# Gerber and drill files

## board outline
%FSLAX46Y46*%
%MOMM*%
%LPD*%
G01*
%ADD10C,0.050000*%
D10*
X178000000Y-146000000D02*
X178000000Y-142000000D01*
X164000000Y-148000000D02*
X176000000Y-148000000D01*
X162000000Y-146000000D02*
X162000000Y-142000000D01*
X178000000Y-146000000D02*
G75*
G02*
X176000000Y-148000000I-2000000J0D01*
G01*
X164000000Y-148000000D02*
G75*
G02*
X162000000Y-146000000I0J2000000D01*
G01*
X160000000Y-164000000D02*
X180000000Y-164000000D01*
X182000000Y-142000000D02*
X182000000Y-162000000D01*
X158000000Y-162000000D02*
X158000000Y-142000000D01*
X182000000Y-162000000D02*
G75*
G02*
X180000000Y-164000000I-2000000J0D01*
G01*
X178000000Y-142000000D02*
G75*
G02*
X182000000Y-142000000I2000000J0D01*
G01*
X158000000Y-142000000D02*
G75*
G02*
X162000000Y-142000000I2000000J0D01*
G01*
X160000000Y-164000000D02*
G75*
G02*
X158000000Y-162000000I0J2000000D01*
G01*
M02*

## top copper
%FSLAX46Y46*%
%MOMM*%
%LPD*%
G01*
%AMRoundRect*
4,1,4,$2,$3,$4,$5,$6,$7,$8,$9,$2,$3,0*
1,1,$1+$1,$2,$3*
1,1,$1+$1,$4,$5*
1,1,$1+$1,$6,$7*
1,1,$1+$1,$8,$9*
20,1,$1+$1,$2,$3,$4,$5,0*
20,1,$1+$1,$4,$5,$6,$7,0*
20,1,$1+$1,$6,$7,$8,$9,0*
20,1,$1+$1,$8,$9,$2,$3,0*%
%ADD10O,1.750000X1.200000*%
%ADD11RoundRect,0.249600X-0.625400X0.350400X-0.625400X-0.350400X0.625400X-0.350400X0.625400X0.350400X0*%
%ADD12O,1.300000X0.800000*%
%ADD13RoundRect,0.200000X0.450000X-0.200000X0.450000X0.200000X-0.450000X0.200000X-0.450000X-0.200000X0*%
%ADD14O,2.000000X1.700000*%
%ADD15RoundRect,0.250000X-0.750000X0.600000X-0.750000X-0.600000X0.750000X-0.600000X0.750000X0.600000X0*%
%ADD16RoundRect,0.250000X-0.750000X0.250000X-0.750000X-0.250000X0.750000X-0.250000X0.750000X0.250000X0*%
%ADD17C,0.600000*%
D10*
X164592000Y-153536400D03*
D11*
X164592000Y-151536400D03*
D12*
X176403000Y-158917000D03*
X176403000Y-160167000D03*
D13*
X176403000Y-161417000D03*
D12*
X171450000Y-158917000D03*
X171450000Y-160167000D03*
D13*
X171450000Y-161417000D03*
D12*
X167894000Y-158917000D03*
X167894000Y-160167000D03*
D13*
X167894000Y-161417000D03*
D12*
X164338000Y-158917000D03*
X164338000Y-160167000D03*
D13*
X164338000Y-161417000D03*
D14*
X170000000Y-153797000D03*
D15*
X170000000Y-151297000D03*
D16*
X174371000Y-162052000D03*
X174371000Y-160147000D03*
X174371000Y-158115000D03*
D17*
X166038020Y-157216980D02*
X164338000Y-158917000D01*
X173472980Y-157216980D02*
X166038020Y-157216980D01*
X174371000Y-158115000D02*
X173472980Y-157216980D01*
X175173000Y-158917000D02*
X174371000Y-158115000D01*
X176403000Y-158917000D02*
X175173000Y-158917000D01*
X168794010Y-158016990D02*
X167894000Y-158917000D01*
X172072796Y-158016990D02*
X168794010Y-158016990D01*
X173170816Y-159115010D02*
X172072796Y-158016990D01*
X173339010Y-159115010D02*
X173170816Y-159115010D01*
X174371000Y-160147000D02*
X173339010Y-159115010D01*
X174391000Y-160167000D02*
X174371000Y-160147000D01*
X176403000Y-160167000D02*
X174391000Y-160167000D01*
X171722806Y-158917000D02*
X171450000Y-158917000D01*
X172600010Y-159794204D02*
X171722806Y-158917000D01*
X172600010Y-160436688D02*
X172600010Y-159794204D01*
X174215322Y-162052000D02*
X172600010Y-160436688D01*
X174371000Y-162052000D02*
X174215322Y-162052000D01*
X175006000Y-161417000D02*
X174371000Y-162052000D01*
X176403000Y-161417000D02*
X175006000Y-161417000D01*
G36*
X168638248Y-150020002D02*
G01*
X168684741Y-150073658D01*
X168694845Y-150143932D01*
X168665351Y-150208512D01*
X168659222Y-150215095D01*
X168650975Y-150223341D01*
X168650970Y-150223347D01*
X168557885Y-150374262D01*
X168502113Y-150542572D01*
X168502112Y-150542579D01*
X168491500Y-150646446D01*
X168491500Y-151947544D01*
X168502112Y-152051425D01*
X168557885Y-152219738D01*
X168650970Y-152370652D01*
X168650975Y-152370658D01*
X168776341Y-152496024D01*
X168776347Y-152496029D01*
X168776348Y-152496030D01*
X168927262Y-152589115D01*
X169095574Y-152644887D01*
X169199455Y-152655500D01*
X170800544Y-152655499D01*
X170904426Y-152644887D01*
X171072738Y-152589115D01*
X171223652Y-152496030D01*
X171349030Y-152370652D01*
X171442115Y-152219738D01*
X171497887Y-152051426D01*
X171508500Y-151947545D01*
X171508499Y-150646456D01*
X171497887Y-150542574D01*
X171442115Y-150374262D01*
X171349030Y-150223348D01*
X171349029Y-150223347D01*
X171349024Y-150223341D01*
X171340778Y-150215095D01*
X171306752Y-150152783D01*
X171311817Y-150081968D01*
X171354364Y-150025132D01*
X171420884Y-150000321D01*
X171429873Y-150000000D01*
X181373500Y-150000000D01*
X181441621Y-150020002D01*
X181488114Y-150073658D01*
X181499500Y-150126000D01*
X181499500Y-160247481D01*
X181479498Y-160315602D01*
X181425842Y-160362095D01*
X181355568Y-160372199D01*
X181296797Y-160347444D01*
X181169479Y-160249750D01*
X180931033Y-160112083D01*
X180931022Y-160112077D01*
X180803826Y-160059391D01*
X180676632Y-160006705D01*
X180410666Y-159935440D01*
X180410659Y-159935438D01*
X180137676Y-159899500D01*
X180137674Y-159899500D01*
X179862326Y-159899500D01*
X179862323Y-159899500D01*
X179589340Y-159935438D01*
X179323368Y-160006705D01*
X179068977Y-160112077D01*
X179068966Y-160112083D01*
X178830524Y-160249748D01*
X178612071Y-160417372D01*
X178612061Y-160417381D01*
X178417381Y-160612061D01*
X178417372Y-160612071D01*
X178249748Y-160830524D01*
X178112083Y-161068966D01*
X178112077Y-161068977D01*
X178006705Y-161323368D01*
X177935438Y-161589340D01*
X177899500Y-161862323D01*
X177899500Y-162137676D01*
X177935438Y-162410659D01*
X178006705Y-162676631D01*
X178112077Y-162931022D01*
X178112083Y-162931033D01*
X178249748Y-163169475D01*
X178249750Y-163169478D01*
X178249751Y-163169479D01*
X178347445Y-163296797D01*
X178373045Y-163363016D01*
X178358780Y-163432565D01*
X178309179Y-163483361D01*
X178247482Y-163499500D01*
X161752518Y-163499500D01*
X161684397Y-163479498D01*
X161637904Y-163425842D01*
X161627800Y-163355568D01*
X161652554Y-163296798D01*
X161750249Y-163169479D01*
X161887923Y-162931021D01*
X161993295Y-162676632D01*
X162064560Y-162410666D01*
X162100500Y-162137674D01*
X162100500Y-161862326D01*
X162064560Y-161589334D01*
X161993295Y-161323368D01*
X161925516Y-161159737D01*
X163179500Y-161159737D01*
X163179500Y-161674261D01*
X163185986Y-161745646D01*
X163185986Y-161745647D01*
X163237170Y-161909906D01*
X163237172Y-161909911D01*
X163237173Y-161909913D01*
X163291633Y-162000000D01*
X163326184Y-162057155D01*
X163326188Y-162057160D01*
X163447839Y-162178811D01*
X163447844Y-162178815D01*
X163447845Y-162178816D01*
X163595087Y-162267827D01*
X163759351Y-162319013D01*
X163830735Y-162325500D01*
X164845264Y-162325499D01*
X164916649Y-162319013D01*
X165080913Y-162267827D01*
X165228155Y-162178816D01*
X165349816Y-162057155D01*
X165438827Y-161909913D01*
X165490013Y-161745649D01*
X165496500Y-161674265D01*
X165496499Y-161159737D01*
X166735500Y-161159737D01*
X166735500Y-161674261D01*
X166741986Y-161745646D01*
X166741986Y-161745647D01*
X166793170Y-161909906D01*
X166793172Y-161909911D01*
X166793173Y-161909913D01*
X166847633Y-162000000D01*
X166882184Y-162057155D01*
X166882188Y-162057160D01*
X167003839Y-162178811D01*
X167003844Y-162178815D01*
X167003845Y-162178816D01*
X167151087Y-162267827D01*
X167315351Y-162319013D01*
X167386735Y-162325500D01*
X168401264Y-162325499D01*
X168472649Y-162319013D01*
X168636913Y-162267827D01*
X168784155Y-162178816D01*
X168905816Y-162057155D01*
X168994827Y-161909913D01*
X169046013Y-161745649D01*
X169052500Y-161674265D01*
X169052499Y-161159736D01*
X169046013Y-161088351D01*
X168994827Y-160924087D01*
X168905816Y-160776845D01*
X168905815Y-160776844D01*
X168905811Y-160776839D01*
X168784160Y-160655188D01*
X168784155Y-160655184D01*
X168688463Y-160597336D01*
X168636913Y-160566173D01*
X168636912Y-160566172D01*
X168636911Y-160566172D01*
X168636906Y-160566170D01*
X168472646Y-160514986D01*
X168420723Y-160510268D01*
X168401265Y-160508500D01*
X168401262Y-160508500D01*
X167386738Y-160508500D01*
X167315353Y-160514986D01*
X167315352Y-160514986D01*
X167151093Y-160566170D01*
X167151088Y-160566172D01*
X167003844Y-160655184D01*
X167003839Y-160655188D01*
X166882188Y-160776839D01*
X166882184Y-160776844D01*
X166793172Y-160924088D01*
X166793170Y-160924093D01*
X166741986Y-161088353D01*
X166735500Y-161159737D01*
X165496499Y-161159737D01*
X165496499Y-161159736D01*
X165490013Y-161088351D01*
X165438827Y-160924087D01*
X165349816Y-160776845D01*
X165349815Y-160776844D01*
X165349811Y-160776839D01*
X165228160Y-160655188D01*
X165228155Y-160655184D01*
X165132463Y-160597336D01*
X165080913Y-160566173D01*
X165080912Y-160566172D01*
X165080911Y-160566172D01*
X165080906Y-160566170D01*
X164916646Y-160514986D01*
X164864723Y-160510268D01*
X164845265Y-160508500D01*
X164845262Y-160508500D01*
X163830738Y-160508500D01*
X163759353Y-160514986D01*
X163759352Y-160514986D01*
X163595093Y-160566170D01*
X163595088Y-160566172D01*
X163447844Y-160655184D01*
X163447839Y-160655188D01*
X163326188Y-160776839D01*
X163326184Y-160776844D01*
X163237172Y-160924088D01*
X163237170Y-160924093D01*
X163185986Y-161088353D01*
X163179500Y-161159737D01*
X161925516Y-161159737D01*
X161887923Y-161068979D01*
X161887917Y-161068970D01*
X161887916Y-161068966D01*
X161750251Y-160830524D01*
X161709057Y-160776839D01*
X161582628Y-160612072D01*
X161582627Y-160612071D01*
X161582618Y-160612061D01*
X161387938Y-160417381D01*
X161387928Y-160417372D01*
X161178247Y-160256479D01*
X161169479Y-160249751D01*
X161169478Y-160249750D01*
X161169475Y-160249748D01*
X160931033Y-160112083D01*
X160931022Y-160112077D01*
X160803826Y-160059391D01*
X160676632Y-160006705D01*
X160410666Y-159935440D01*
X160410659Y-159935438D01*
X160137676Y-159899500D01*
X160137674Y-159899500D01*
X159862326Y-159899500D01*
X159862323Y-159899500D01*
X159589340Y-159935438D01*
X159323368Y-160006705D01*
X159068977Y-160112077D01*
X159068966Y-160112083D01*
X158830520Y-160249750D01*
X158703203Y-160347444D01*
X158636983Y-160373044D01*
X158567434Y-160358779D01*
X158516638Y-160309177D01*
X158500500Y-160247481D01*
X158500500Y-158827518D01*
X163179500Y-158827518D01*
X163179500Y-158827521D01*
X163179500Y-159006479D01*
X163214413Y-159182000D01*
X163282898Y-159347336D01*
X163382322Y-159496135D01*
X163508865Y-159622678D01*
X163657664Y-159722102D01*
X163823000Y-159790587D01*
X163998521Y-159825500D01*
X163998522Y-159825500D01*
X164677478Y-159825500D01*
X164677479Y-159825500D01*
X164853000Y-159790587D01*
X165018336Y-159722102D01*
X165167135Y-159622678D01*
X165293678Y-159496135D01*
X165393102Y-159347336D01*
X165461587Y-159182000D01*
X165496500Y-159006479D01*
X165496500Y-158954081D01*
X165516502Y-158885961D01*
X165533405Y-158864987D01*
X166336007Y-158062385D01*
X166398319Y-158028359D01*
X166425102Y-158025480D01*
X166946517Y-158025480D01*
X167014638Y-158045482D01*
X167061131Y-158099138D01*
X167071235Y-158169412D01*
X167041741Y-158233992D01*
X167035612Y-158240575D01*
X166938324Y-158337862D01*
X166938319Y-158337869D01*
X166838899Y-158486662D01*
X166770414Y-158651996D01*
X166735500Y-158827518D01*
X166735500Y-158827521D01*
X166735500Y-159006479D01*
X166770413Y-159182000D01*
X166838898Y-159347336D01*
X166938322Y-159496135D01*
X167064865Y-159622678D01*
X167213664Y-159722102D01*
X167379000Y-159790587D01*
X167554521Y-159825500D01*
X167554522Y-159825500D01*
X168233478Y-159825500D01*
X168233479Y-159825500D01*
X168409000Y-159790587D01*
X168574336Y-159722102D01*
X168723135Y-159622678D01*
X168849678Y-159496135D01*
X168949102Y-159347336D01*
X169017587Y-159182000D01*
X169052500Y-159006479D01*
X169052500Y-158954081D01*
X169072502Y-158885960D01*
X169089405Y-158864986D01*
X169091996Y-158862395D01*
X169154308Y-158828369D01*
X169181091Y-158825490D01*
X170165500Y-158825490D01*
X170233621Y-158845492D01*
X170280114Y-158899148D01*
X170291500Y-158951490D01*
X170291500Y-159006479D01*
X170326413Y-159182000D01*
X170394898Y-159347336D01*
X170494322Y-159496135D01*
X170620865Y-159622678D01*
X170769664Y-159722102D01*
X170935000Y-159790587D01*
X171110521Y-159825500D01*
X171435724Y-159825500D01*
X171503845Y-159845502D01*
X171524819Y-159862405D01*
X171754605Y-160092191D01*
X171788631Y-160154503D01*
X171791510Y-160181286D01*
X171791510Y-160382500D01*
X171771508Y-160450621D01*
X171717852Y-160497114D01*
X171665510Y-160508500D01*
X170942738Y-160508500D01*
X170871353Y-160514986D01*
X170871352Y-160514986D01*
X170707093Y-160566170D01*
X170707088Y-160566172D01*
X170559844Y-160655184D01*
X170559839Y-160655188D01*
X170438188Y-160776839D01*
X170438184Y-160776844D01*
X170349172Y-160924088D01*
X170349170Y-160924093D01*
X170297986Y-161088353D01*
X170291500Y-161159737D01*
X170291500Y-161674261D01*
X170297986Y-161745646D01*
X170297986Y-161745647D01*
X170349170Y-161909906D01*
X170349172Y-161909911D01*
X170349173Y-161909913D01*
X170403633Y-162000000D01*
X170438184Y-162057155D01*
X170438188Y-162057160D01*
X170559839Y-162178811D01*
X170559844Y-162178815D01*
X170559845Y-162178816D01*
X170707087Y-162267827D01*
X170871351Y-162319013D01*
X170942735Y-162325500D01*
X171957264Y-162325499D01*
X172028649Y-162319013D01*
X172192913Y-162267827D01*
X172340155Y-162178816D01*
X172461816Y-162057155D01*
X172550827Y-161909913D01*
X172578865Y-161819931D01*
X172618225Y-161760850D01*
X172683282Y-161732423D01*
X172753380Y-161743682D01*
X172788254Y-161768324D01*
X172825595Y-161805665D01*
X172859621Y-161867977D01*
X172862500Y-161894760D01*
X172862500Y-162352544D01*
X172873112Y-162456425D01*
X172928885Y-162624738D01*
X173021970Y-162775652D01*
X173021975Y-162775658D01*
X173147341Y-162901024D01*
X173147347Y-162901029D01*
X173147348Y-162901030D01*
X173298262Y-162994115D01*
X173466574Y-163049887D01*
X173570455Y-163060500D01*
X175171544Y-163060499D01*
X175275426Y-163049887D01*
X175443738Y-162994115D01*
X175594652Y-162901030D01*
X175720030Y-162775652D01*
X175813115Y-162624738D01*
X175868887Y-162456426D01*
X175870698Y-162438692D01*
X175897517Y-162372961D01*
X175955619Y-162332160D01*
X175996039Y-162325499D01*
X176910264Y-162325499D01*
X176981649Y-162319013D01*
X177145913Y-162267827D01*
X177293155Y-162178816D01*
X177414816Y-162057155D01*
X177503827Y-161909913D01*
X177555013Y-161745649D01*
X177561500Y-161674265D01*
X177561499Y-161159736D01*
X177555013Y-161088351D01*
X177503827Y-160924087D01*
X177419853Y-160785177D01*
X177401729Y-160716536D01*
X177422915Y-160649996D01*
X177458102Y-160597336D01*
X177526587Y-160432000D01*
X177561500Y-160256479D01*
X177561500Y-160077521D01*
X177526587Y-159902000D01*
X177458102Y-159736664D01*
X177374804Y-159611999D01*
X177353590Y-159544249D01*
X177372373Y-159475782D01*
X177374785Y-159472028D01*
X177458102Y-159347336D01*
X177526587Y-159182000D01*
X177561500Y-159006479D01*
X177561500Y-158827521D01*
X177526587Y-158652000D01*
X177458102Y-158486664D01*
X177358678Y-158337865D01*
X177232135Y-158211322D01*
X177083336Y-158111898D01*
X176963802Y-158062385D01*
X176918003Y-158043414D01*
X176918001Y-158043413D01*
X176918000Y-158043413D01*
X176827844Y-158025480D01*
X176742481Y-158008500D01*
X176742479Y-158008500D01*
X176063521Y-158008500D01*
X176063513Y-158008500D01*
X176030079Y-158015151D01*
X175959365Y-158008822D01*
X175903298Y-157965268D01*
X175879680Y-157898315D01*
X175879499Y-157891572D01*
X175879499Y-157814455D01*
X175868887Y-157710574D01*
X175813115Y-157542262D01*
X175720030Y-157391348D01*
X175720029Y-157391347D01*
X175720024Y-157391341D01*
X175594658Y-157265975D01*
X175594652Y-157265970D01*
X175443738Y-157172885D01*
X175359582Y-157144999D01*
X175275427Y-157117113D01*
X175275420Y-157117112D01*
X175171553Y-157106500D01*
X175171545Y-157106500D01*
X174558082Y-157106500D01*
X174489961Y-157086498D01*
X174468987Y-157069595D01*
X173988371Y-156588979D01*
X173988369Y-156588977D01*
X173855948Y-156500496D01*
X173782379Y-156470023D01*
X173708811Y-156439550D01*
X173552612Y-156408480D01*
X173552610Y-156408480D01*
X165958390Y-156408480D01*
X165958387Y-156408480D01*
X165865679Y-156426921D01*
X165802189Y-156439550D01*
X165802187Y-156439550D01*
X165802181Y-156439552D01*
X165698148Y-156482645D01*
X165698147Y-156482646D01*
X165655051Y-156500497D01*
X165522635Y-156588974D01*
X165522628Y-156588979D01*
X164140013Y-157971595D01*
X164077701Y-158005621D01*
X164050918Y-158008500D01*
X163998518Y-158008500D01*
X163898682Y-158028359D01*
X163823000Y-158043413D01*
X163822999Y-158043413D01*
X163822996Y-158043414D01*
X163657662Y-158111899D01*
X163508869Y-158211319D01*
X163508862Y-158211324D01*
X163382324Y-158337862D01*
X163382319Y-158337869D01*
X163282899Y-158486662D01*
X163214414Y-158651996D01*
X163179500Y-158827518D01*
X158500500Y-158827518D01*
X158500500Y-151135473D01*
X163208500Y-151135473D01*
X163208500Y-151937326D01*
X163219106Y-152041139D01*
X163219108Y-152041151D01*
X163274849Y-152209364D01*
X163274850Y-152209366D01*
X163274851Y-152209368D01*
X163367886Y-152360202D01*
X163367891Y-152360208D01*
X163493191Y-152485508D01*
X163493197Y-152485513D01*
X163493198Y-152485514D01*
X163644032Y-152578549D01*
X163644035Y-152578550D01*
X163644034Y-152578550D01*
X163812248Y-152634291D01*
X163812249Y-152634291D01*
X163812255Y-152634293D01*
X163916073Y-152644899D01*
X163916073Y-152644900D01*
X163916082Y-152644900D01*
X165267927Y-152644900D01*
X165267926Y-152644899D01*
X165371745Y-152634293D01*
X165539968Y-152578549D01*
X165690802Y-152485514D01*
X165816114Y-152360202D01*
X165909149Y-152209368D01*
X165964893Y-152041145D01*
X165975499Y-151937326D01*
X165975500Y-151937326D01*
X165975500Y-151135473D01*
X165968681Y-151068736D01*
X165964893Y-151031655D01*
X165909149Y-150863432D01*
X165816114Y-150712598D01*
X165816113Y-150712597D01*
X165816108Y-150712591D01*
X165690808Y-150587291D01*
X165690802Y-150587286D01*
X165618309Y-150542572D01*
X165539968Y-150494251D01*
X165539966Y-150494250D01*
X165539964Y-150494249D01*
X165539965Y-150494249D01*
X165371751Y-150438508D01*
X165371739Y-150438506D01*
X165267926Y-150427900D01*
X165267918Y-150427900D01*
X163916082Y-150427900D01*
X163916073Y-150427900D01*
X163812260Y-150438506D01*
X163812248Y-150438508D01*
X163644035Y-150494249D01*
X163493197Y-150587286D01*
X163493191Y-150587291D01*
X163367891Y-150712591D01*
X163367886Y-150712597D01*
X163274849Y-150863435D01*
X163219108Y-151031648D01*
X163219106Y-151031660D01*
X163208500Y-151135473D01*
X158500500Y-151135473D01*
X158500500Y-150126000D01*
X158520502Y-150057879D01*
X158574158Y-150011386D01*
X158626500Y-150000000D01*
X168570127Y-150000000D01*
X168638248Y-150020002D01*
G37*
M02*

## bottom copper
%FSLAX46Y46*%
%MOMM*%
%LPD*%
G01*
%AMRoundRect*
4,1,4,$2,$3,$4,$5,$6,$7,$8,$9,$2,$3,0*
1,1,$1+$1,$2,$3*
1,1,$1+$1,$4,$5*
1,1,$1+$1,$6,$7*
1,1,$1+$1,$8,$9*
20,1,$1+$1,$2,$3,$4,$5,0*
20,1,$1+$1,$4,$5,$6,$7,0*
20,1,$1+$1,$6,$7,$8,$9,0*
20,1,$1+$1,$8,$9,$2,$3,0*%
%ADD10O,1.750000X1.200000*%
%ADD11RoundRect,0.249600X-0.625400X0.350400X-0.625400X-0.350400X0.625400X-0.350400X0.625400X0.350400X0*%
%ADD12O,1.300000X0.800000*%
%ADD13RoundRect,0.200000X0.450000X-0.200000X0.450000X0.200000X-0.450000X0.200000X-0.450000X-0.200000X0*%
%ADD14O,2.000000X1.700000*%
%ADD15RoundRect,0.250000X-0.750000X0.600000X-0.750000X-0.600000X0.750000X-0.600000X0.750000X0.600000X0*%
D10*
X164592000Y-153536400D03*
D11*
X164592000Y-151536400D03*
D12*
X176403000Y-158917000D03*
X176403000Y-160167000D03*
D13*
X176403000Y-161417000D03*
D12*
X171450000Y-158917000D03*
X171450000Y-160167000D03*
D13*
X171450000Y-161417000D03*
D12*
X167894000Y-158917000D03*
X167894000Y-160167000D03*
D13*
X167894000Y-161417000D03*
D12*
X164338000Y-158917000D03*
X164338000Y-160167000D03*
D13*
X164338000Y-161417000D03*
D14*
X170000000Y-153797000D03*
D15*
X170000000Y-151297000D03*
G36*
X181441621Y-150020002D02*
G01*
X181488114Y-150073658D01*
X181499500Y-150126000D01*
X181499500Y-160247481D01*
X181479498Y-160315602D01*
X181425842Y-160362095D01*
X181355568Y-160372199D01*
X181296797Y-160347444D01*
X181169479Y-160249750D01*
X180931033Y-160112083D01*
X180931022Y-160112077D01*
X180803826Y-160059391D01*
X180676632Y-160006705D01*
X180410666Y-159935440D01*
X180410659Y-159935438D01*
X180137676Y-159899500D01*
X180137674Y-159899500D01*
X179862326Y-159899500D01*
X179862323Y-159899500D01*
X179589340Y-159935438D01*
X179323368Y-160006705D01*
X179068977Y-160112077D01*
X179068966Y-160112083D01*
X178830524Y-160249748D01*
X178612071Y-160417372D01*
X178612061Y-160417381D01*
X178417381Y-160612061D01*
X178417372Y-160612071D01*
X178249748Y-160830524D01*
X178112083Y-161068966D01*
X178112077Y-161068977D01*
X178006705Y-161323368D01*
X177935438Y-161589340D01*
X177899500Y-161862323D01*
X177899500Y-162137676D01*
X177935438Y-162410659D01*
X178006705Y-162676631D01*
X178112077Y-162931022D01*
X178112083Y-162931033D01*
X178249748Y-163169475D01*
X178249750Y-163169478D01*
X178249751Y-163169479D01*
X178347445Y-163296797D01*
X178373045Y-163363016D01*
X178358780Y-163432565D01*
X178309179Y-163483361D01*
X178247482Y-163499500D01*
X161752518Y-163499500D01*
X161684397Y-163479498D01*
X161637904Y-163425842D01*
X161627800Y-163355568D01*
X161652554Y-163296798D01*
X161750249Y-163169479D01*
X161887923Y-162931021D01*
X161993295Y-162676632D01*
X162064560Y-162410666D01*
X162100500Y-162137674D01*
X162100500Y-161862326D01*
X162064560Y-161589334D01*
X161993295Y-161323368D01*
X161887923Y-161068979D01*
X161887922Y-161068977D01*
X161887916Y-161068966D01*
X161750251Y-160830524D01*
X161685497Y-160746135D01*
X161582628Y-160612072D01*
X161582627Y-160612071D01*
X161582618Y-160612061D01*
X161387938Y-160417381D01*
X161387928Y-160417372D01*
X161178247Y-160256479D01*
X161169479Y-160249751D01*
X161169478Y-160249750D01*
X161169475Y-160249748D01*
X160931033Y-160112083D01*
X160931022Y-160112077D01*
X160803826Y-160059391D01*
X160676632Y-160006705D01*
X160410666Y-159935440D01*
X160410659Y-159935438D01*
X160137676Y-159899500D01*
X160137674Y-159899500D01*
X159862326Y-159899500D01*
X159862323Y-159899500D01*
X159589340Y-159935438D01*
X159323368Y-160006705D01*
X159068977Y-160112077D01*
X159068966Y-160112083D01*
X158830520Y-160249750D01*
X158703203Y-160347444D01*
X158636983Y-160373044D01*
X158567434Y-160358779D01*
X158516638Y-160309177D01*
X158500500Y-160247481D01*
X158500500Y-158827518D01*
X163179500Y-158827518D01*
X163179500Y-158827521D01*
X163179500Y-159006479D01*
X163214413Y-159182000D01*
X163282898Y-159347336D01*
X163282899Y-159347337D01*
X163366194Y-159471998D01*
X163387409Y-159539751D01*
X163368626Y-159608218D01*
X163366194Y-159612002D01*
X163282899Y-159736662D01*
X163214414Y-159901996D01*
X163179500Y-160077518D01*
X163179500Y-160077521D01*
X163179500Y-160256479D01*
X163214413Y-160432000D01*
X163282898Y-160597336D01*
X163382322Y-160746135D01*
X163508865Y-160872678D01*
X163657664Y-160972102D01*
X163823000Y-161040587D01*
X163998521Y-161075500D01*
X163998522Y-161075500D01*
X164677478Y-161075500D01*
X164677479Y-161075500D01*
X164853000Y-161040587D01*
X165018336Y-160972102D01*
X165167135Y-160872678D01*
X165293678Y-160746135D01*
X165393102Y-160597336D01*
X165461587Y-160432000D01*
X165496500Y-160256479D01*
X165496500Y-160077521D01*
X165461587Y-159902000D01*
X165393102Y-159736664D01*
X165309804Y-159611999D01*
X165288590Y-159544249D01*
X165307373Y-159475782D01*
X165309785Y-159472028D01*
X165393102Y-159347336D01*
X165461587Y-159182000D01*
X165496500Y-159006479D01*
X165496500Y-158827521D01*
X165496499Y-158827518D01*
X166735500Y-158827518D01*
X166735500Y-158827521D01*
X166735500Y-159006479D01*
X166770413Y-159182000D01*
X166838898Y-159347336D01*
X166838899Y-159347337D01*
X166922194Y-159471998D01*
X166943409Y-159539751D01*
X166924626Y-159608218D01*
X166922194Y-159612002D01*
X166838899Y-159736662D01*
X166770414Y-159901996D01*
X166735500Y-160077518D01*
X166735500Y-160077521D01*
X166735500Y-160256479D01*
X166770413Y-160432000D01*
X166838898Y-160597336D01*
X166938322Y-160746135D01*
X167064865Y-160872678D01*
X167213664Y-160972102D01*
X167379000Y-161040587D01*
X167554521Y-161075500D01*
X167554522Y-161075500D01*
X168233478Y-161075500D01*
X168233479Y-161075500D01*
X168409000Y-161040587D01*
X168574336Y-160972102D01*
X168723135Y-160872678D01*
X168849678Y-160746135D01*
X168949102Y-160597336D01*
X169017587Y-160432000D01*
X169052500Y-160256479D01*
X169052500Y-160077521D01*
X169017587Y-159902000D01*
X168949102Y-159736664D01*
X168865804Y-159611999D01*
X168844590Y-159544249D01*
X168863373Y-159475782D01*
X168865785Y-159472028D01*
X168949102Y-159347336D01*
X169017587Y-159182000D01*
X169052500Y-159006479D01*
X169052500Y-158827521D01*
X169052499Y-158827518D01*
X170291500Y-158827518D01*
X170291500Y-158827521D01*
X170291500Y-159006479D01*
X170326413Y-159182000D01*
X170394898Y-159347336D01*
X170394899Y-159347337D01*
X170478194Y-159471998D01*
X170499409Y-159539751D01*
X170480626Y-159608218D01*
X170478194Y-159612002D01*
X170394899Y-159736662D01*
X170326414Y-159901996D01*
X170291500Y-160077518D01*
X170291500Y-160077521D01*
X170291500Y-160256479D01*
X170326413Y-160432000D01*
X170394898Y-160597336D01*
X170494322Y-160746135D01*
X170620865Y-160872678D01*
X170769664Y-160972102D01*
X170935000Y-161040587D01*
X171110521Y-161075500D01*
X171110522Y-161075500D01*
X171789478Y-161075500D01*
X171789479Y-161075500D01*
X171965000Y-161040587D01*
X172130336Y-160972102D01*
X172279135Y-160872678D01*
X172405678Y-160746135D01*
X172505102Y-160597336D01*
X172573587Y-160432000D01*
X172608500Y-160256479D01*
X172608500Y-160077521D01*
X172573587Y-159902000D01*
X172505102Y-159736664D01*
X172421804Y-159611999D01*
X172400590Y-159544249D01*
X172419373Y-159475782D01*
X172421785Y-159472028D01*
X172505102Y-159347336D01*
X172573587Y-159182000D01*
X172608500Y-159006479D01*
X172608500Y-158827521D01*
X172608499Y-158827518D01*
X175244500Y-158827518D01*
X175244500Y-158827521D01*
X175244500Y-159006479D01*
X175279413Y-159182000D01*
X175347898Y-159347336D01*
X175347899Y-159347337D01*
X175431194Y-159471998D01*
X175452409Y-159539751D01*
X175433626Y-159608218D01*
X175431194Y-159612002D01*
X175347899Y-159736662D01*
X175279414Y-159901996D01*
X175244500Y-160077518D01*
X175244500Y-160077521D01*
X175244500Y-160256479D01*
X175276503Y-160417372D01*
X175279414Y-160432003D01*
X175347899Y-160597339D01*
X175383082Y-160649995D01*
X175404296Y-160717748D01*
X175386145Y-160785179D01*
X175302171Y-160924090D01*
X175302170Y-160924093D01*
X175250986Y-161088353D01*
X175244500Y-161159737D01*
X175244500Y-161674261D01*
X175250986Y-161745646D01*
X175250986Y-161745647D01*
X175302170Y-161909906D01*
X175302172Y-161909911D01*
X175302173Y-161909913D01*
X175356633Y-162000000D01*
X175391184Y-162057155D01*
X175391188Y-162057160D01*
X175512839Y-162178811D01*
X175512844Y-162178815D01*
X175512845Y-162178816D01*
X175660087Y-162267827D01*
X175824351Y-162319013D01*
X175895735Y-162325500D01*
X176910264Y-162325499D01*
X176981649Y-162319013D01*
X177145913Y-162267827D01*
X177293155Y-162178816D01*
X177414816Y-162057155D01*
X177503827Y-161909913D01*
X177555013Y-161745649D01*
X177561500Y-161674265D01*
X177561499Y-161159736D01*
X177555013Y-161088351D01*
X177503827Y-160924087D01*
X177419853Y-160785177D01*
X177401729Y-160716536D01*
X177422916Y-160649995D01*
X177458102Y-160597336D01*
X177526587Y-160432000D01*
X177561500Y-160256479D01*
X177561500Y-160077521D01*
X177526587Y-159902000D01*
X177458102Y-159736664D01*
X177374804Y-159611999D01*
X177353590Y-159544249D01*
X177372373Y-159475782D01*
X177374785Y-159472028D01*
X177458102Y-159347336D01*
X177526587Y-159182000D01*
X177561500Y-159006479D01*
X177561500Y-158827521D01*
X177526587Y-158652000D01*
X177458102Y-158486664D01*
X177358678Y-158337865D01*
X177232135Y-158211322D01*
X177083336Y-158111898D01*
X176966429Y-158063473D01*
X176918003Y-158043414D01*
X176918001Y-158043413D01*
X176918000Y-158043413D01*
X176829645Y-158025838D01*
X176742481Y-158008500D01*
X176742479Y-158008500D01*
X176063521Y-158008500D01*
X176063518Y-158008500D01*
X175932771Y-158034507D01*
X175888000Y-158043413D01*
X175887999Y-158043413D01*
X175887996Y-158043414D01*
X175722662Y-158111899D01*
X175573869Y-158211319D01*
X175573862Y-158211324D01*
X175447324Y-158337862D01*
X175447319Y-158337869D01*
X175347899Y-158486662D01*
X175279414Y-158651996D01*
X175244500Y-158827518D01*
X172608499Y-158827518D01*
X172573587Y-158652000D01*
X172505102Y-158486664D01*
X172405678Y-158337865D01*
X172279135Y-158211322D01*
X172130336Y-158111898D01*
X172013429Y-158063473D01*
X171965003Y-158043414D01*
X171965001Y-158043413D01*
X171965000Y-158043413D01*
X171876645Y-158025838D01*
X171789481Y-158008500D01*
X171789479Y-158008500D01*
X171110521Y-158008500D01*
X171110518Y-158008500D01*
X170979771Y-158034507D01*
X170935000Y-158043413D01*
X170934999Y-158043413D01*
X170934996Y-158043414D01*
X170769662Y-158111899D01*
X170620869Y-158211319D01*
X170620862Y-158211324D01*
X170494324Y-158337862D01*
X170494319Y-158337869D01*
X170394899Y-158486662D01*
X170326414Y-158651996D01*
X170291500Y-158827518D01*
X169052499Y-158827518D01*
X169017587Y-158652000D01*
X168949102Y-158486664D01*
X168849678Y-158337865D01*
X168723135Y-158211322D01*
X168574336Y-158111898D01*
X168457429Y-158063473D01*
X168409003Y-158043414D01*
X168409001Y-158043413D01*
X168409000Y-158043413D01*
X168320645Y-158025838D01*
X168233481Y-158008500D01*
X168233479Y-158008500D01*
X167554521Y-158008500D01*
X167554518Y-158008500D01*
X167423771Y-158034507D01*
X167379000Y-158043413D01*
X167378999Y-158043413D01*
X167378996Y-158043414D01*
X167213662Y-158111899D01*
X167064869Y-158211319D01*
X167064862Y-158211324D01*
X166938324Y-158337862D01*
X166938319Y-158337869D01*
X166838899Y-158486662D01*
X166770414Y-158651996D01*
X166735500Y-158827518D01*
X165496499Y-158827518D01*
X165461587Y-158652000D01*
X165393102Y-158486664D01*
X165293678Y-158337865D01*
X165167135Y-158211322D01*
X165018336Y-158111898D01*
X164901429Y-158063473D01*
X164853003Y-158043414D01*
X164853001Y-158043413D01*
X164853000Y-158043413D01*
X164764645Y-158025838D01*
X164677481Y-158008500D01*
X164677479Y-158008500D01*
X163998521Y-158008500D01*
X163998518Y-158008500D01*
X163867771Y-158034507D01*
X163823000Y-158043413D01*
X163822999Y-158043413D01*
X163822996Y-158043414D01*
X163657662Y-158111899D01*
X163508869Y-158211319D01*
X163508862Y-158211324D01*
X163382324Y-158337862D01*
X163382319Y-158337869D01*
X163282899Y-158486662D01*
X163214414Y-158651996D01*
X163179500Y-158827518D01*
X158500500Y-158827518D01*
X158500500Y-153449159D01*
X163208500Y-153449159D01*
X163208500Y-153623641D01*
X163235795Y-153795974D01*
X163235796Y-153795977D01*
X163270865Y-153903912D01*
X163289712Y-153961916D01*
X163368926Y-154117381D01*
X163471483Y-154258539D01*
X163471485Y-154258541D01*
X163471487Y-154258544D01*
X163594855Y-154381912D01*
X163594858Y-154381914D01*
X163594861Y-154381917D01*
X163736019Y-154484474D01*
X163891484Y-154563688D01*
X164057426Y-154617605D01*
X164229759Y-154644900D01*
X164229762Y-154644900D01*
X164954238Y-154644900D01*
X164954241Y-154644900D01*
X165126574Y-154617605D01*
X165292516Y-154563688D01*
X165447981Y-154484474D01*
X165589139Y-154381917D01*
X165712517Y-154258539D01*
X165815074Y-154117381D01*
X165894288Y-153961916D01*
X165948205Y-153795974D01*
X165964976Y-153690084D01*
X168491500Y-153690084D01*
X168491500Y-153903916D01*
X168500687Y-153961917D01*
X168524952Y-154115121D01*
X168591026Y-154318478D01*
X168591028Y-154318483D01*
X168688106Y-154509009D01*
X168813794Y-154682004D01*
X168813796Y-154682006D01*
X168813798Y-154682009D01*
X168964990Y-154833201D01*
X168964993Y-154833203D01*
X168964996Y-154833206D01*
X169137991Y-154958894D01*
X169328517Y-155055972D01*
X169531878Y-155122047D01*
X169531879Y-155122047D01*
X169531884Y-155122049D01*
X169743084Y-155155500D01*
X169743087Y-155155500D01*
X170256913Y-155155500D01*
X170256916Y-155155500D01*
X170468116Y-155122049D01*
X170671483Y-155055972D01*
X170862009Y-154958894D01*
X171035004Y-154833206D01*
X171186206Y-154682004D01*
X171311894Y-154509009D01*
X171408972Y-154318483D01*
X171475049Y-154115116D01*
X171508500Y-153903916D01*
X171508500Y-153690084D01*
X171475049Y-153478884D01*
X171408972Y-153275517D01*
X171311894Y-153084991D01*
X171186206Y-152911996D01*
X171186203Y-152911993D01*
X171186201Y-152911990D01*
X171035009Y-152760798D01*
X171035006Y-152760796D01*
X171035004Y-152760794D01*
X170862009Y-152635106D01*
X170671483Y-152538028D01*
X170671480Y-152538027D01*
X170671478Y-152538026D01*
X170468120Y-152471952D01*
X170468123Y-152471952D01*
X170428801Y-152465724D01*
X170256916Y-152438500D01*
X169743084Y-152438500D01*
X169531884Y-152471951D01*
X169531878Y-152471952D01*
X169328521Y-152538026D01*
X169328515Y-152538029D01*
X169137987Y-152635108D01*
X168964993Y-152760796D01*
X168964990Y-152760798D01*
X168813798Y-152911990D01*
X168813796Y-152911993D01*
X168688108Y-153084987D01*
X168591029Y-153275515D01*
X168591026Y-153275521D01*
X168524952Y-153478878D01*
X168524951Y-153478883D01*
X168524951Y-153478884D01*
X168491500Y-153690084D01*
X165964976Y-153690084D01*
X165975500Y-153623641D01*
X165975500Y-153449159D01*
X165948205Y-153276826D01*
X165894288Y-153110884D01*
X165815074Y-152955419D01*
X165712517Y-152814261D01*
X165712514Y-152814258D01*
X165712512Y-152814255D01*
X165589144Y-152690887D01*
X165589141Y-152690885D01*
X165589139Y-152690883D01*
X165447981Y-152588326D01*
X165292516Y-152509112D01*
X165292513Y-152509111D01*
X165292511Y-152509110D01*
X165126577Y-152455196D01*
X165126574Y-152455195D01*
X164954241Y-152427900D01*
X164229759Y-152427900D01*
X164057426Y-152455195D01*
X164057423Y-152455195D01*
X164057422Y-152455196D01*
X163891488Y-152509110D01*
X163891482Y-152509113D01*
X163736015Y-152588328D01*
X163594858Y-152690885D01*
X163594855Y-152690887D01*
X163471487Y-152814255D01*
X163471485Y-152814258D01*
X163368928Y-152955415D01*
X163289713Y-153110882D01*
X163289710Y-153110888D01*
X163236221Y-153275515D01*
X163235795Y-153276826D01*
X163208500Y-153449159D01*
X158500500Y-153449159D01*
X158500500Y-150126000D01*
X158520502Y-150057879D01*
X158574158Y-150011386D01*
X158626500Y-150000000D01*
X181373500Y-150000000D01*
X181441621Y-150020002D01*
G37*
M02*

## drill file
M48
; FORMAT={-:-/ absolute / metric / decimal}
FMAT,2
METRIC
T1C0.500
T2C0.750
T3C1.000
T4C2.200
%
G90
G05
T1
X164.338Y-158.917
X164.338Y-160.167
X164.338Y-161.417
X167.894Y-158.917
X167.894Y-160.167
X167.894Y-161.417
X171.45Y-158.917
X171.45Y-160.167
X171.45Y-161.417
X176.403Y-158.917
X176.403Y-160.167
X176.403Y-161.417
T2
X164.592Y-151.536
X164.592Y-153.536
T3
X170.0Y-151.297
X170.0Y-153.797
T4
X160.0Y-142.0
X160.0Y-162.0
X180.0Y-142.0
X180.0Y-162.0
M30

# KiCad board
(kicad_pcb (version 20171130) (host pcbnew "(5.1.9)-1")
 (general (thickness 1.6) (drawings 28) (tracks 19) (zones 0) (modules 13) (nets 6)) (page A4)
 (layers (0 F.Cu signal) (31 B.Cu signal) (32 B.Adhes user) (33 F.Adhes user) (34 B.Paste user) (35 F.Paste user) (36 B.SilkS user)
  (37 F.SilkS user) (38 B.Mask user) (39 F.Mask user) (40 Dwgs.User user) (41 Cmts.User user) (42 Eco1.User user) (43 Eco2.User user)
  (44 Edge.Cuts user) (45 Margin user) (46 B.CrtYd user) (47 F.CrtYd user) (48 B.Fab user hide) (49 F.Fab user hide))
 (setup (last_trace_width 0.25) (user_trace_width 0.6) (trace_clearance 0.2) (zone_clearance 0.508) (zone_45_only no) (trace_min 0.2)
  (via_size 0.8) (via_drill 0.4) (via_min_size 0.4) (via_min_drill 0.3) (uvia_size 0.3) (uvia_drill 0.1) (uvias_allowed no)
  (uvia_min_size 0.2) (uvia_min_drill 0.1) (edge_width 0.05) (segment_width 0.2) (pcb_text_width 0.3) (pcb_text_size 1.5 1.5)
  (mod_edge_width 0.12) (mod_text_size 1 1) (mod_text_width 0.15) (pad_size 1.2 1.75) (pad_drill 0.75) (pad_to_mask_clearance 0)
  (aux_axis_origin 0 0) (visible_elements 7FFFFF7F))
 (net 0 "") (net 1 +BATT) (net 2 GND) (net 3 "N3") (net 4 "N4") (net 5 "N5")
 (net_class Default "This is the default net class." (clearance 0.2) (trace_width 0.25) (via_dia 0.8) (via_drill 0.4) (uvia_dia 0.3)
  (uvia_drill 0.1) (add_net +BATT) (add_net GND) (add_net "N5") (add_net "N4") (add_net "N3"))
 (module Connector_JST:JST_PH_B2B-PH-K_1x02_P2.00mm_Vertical (layer B.Cu) (at 164.592 151.5364 270)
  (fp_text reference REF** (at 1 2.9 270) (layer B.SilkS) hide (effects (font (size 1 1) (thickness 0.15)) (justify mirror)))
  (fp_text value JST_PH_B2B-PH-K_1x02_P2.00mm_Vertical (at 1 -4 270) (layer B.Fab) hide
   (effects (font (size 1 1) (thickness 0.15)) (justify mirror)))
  (pad 2 thru_hole oval (at 2 0 270) (size 1.2 1.75) (drill 0.75) (layers *.Cu *.Mask) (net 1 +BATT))
  (pad 1 thru_hole roundrect (at 0 0 270) (size 1.2 1.75) (drill 0.75) (layers *.Cu *.Mask) (roundrect_rratio 0.208) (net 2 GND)))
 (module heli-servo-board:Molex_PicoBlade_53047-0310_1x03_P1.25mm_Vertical (layer F.Cu) (at 176.403 161.417 90)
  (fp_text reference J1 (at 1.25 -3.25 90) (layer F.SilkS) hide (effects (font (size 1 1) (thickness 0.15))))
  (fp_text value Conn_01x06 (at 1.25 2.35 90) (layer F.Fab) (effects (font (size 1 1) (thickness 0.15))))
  (pad 3 thru_hole oval (at 2.5 0 90) (size 0.8 1.3) (drill 0.5) (layers *.Cu *.Mask) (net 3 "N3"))
  (pad 2 thru_hole oval (at 1.25 0 90) (size 0.8 1.3) (drill 0.5) (layers *.Cu *.Mask) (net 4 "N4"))
  (pad 1 thru_hole roundrect (at 0 0 90) (size 0.8 1.3) (drill 0.5) (layers *.Cu *.Mask) (roundrect_rratio 0.25) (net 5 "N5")))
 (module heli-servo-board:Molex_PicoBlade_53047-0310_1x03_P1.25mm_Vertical (layer F.Cu) (at 171.45 161.417 90)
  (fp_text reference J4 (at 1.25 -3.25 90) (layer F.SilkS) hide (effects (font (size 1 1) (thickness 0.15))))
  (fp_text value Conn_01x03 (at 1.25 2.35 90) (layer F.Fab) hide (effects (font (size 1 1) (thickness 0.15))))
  (pad 3 thru_hole oval (at 2.5 0 90) (size 0.8 1.3) (drill 0.5) (layers *.Cu *.Mask) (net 5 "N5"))
  (pad 2 thru_hole oval (at 1.25 0 90) (size 0.8 1.3) (drill 0.5) (layers *.Cu *.Mask) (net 1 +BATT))
  (pad 1 thru_hole roundrect (at 0 0 90) (size 0.8 1.3) (drill 0.5) (layers *.Cu *.Mask) (roundrect_rratio 0.25) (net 2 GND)))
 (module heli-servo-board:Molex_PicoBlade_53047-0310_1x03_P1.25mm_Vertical (layer F.Cu) (at 167.894 161.417 90)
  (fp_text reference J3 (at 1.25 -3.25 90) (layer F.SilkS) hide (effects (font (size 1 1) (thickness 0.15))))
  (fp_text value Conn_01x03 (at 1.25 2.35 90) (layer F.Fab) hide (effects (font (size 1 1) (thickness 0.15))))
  (pad 3 thru_hole oval (at 2.5 0 90) (size 0.8 1.3) (drill 0.5) (layers *.Cu *.Mask) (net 4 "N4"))
  (pad 2 thru_hole oval (at 1.25 0 90) (size 0.8 1.3) (drill 0.5) (layers *.Cu *.Mask) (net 1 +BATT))
  (pad 1 thru_hole roundrect (at 0 0 90) (size 0.8 1.3) (drill 0.5) (layers *.Cu *.Mask) (roundrect_rratio 0.25) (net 2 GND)))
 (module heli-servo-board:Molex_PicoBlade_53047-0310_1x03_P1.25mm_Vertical (layer F.Cu) (at 164.338 161.417 90)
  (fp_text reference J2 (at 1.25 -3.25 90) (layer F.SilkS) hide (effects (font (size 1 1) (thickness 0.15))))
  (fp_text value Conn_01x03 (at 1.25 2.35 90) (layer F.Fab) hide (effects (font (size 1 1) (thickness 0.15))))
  (pad 3 thru_hole oval (at 2.5 0 90) (size 0.8 1.3) (drill 0.5) (layers *.Cu *.Mask) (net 3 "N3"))
  (pad 2 thru_hole oval (at 1.25 0 90) (size 0.8 1.3) (drill 0.5) (layers *.Cu *.Mask) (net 1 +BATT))
  (pad 1 thru_hole roundrect (at 0 0 90) (size 0.8 1.3) (drill 0.5) (layers *.Cu *.Mask) (roundrect_rratio 0.25) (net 2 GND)))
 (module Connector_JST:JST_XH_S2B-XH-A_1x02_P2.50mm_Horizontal (layer F.Cu) (at 170 151.297 270)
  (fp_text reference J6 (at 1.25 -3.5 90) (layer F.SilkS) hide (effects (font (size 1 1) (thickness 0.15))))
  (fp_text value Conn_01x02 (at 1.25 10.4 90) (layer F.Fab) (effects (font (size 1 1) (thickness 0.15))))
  (pad 2 thru_hole oval (at 2.5 0 270) (size 1.7 2) (drill 1) (layers *.Cu *.Mask) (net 1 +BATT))
  (pad 1 thru_hole roundrect (at 0 0 270) (size 1.7 2) (drill 1) (layers *.Cu *.Mask) (roundrect_rratio 0.1470588235294118) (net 2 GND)))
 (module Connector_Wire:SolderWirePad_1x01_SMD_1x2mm (layer F.Cu) (at 174.371 162.052 270)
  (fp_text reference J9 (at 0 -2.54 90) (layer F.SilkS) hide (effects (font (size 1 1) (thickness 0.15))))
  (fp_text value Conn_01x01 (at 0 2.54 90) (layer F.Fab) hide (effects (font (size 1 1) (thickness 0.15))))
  (pad 1 smd roundrect (at 0 0 270) (size 1 2) (layers F.Cu F.Paste F.Mask) (roundrect_rratio 0.25) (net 5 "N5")))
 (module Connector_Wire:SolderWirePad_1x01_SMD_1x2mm (layer F.Cu) (at 174.371 160.147 270)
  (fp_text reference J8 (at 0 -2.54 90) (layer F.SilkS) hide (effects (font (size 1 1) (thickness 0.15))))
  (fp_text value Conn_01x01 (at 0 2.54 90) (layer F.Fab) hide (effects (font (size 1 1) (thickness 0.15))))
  (pad 1 smd roundrect (at 0 0 270) (size 1 2) (layers F.Cu F.Paste F.Mask) (roundrect_rratio 0.25) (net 4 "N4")))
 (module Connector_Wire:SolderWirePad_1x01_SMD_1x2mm (layer F.Cu) (at 174.371 158.115 270)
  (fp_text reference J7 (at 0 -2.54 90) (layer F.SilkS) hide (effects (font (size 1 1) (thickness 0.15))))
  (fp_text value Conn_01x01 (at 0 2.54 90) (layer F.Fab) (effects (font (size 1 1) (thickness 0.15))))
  (pad 1 smd roundrect (at 0 0 270) (size 1 2) (layers F.Cu F.Paste F.Mask) (roundrect_rratio 0.25) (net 3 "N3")))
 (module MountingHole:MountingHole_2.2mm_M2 (layer F.Cu) (at 180 162)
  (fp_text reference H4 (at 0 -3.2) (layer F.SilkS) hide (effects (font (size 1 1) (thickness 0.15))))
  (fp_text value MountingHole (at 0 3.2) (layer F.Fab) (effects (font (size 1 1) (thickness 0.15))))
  (pad "" np_thru_hole circle (at 0 0) (size 2.2 2.2) (drill 2.2) (layers *.Cu *.Mask) (clearance 1)))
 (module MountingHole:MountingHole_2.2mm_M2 (layer F.Cu) (at 180 142)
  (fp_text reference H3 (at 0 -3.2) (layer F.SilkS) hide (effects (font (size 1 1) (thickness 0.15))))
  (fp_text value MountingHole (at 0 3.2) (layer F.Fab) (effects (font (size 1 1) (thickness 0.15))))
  (pad "" np_thru_hole circle (at 0 0) (size 2.2 2.2) (drill 2.2) (layers *.Cu *.Mask) (clearance 1)))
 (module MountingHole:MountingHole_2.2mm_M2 (layer F.Cu) (at 160 162)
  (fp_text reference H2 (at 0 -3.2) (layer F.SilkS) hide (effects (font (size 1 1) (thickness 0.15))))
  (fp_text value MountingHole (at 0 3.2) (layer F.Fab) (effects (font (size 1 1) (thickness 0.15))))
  (pad "" np_thru_hole circle (at 0 0) (size 2.2 2.2) (drill 2.2) (layers *.Cu *.Mask) (clearance 1)))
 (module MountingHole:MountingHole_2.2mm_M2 (layer F.Cu) (at 160 142)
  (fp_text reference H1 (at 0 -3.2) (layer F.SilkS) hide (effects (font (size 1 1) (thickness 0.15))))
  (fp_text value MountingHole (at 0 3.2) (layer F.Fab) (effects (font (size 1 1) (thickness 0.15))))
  (pad "" np_thru_hole circle (at 0 0) (size 2.2 2.2) (drill 2.2) (layers *.Cu *.Mask) (clearance 1)))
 (gr_line (start 178 146) (end 178 142) (layer Edge.Cuts) (width 0.05))
 (gr_line (start 164 148) (end 176 148) (layer Edge.Cuts) (width 0.05))
 (gr_line (start 162 146) (end 162 142) (layer Edge.Cuts) (width 0.05))
 (gr_arc (start 176 146) (end 176 148) (angle -90) (layer Edge.Cuts) (width 0.05))
 (gr_arc (start 164 146) (end 162 146) (angle -90) (layer Edge.Cuts) (width 0.05))
 (gr_line (start 160 164) (end 180 164) (layer Edge.Cuts) (width 0.05))
 (gr_line (start 182 142) (end 182 162) (layer Edge.Cuts) (width 0.05))
 (gr_line (start 158 162) (end 158 142) (layer Edge.Cuts) (width 0.05))
 (gr_arc (start 180 162) (end 180 164) (angle -90) (layer Edge.Cuts) (width 0.05))
 (gr_arc (start 180 142) (end 182 142) (angle -180) (layer Edge.Cuts) (width 0.05))
 (gr_arc (start 160 142) (end 162 142) (angle -180) (layer Edge.Cuts) (width 0.05))
 (gr_arc (start 160 162) (end 158 162) (angle -90) (layer Edge.Cuts) (width 0.05))
 (segment (start 166.03802 157.21698) (end 164.338 158.917) (width 0.6) (layer F.Cu) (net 3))
 (segment (start 173.47298 157.21698) (end 166.03802 157.21698) (width 0.6) (layer F.Cu) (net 3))
 (segment (start 174.371 158.115) (end 173.47298 157.21698) (width 0.6) (layer F.Cu) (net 3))
 (segment (start 175.173 158.917) (end 174.371 158.115) (width 0.6) (layer F.Cu) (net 3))
 (segment (start 176.403 158.917) (end 175.173 158.917) (width 0.6) (layer F.Cu) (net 3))
 (segment (start 168.79401 158.01699) (end 167.894 158.917) (width 0.6) (layer F.Cu) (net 4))
 (segment (start 172.072796 158.01699) (end 168.79401 158.01699) (width 0.6) (layer F.Cu) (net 4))
 (segment (start 173.170816 159.11501) (end 172.072796 158.01699) (width 0.6) (layer F.Cu) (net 4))
 (segment (start 173.33901 159.11501) (end 173.170816 159.11501) (width 0.6) (layer F.Cu) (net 4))
 (segment (start 174.371 160.147) (end 173.33901 159.11501) (width 0.6) (layer F.Cu) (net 4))
 (segment (start 174.391 160.167) (end 174.371 160.147) (width 0.6) (layer F.Cu) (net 4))
 (segment (start 176.403 160.167) (end 174.391 160.167) (width 0.6) (layer F.Cu) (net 4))
 (segment (start 171.722806 158.917) (end 171.45 158.917) (width 0.6) (layer F.Cu) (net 5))
 (segment (start 172.60001 159.794204) (end 171.722806 158.917) (width 0.6) (layer F.Cu) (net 5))
 (segment (start 172.60001 160.436688) (end 172.60001 159.794204) (width 0.6) (layer F.Cu) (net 5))
 (segment (start 174.215322 162.052) (end 172.60001 160.436688) (width 0.6) (layer F.Cu) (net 5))
 (segment (start 174.371 162.052) (end 174.215322 162.052) (width 0.6) (layer F.Cu) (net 5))
 (segment (start 175.006 161.417) (end 174.371 162.052) (width 0.6) (layer F.Cu) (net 5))
 (segment (start 176.403 161.417) (end 175.006 161.417) (width 0.6) (layer F.Cu) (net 5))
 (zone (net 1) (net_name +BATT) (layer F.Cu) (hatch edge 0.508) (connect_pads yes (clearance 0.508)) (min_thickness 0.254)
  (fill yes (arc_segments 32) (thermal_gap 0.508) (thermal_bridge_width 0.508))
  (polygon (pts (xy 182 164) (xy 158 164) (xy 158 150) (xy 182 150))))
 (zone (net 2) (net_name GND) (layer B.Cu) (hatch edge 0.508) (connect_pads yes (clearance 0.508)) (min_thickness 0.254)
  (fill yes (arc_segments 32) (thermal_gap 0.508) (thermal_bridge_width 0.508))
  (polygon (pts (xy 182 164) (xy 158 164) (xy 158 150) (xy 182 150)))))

